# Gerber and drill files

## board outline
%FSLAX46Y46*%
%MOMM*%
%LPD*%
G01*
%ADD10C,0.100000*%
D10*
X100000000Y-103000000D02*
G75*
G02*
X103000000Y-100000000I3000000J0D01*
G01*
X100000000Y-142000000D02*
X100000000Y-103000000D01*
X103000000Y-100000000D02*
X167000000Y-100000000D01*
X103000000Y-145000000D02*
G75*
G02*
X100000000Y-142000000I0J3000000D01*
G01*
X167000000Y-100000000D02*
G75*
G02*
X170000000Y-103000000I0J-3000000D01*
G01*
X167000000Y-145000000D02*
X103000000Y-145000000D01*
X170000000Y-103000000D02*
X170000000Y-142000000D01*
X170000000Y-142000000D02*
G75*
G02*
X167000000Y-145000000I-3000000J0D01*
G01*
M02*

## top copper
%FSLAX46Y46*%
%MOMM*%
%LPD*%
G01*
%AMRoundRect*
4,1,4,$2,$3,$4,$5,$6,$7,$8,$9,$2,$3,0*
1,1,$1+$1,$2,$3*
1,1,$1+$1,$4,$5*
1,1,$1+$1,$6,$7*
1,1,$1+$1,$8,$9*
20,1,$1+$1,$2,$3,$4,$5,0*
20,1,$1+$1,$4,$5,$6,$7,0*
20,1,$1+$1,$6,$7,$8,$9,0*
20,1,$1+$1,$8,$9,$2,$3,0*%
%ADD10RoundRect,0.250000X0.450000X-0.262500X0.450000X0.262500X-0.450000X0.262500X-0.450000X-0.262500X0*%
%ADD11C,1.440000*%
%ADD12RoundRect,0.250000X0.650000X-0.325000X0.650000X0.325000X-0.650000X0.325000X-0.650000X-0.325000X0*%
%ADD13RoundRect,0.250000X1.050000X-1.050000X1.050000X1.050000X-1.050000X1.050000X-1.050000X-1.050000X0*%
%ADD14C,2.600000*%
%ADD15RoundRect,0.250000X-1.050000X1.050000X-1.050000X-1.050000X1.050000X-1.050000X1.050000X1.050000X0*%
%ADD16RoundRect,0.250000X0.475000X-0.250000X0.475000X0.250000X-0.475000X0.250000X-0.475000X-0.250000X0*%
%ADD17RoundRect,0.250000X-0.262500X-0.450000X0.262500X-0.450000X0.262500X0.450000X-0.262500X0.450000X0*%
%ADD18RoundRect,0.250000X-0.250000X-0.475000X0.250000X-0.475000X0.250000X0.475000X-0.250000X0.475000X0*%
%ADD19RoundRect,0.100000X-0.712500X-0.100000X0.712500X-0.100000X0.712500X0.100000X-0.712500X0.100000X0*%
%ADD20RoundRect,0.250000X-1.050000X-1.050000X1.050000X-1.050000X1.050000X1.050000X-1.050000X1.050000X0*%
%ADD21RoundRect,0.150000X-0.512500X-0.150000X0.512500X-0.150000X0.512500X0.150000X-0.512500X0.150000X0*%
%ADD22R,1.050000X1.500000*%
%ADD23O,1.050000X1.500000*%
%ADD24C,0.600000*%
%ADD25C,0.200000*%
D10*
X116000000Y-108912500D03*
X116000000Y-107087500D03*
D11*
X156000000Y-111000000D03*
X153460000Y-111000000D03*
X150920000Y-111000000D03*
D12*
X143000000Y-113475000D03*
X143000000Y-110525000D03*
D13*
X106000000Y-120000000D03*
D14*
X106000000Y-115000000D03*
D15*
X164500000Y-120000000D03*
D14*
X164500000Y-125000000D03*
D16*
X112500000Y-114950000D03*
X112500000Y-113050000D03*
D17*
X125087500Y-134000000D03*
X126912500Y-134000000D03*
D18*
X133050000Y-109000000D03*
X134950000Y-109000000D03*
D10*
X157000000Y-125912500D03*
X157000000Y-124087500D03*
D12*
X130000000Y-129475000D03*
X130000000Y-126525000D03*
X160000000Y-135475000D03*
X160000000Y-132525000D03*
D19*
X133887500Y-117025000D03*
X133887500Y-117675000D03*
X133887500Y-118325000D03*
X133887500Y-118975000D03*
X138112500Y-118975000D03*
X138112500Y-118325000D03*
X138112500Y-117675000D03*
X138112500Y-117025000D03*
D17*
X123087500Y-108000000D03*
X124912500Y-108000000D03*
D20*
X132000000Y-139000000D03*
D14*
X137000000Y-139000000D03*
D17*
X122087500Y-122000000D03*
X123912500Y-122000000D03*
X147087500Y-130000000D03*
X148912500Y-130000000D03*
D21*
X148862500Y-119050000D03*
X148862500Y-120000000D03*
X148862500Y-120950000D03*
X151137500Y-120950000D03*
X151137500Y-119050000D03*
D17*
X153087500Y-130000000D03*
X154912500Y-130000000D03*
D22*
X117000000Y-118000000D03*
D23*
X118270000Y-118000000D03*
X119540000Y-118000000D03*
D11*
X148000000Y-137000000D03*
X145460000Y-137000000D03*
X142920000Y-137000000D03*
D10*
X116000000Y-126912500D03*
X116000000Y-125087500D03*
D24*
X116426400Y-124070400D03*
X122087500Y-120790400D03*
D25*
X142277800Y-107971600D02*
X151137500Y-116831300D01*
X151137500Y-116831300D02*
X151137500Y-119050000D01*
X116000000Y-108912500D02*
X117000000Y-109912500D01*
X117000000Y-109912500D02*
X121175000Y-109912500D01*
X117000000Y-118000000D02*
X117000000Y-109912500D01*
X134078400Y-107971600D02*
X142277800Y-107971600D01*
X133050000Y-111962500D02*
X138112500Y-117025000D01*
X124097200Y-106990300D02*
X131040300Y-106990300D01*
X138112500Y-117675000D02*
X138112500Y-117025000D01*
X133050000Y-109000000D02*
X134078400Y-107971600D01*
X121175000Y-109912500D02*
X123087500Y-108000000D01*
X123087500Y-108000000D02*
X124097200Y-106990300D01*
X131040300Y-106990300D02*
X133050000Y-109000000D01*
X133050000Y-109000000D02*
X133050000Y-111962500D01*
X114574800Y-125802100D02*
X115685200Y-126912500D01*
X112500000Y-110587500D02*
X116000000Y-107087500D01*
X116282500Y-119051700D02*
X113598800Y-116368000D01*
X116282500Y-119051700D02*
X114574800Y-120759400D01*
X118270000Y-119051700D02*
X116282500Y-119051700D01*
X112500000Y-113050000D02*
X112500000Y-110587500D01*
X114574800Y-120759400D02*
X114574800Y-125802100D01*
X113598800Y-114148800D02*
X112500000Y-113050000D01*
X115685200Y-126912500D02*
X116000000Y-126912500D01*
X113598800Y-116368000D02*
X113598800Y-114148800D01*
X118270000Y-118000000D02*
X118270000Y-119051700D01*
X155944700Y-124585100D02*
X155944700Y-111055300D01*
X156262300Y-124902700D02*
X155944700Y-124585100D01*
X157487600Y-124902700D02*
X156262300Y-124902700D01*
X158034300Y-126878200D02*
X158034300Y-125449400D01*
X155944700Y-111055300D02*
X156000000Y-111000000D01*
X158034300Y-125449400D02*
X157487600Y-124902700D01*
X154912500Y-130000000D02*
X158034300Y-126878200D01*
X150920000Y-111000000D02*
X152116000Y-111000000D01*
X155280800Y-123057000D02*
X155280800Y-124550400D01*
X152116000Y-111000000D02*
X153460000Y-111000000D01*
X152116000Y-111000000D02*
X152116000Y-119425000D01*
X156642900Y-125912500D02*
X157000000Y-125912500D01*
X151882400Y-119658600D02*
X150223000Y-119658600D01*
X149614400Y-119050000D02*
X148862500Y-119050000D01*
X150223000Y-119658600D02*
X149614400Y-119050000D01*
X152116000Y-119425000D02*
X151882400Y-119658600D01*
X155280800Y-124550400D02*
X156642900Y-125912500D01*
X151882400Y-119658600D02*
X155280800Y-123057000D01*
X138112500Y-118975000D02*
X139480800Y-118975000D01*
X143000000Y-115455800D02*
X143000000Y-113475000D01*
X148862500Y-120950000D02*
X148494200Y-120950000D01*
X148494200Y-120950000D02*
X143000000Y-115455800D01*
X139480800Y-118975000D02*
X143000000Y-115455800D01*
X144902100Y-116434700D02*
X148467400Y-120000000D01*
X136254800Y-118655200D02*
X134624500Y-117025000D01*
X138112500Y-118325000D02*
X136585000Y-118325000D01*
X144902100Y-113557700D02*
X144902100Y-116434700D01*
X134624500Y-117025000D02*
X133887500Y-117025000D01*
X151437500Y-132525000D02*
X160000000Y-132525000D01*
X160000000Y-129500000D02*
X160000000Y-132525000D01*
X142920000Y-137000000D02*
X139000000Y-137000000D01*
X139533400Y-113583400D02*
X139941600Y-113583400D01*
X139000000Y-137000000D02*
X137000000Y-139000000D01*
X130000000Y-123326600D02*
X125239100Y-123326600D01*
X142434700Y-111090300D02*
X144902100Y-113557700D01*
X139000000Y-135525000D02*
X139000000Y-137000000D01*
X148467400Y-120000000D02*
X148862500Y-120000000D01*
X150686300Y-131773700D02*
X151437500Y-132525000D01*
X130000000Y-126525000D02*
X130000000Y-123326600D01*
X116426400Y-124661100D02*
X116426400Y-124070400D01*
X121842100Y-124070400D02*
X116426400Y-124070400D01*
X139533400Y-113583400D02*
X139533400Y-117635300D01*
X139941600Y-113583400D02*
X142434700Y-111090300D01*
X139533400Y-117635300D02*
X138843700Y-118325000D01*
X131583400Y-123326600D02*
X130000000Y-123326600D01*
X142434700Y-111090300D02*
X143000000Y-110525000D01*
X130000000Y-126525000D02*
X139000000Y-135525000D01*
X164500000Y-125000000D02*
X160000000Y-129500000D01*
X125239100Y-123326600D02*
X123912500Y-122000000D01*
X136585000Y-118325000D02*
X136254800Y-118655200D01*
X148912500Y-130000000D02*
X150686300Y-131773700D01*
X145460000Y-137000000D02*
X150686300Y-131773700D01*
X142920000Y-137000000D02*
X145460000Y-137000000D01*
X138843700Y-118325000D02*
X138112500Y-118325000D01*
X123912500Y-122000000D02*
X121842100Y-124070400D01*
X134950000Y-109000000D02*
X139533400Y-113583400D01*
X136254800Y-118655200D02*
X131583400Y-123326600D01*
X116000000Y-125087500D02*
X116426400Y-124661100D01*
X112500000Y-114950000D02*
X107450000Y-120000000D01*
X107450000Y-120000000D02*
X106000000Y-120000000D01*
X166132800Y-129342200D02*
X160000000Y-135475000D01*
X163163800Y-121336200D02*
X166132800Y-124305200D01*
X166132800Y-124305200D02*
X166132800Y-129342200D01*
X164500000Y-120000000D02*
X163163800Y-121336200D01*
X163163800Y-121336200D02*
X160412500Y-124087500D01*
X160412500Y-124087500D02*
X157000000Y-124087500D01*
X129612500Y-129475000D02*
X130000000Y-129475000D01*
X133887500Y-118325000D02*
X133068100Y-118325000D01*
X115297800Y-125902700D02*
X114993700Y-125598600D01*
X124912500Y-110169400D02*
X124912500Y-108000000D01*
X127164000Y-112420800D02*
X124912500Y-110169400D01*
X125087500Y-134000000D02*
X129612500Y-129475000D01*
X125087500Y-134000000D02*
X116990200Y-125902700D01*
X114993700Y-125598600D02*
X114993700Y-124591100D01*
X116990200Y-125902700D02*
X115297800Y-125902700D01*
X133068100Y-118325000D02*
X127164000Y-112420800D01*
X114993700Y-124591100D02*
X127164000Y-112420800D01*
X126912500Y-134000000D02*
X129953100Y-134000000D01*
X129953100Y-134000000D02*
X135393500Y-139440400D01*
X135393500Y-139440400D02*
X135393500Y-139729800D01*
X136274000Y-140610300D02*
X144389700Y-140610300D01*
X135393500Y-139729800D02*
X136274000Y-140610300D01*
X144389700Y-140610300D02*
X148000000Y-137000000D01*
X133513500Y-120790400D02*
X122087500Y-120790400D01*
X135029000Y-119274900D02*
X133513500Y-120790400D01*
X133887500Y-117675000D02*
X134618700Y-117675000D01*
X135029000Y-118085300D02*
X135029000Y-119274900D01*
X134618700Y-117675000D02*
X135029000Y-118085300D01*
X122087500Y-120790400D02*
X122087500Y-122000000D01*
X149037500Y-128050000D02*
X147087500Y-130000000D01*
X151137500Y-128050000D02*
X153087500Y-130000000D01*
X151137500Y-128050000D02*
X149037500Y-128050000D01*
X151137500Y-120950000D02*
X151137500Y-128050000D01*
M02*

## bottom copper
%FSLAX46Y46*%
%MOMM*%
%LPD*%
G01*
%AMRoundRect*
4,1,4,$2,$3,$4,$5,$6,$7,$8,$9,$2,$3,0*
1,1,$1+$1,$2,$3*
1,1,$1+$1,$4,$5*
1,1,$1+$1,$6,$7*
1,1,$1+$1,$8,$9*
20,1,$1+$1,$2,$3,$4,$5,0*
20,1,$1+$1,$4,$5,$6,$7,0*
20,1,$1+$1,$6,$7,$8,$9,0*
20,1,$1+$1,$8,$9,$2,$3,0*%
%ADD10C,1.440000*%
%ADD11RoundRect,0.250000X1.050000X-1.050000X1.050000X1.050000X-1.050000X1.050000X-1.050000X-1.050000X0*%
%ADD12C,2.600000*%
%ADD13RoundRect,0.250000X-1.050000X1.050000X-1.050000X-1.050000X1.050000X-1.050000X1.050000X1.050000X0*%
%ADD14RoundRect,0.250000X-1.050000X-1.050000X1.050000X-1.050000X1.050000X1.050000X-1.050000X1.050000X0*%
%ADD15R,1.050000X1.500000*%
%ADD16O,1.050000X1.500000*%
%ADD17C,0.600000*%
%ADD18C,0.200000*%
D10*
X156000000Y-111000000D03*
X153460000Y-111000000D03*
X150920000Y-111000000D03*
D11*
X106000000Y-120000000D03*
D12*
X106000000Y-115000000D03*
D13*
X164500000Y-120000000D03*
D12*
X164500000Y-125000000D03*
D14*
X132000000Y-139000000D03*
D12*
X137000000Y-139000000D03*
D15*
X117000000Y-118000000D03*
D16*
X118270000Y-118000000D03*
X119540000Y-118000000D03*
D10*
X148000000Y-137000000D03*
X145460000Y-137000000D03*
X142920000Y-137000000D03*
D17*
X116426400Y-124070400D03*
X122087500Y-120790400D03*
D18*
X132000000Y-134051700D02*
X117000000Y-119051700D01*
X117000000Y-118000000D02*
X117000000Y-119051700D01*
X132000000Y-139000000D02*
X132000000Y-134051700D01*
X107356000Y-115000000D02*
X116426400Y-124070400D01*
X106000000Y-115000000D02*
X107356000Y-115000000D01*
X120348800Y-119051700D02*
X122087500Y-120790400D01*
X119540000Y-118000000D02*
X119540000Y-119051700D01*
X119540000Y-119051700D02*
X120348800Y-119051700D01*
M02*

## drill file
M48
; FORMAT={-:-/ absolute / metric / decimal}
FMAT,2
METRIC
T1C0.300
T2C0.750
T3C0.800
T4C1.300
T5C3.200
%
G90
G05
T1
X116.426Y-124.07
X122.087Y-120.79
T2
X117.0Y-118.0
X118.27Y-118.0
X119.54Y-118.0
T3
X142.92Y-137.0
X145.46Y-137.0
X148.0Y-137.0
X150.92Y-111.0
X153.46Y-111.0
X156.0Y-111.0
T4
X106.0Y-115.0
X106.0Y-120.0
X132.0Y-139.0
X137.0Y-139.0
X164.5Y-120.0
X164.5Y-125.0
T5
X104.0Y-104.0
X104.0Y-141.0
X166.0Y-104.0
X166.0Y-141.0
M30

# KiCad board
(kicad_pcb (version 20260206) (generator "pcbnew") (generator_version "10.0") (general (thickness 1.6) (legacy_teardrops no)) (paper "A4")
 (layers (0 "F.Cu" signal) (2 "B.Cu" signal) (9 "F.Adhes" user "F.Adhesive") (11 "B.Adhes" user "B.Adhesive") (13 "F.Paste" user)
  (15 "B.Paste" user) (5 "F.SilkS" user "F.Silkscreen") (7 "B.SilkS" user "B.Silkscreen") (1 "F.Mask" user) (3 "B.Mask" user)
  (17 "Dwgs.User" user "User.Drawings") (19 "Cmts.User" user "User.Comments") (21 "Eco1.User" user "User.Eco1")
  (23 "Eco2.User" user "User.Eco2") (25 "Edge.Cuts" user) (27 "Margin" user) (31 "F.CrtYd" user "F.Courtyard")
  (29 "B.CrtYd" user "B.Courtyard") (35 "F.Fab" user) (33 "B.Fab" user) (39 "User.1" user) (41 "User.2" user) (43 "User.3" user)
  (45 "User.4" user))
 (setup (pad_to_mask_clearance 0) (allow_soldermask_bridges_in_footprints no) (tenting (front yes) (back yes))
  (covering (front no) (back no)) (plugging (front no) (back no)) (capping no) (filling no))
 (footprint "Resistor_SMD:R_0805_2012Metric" (layer "F.Cu") (at 116 108 90)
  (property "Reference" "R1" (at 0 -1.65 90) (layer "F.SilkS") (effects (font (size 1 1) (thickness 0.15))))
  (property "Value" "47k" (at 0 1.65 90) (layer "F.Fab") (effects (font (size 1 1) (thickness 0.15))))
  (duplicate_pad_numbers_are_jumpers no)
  (pad "1" smd roundrect (at -0.9125 0 90) (size 1.025 1.4) (layers "F.Cu" "F.Mask" "F.Paste") (roundrect_rratio 0.243902) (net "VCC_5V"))
  (pad "2" smd roundrect (at 0.9125 0 90) (size 1.025 1.4) (layers "F.Cu" "F.Mask" "F.Paste") (roundrect_rratio 0.243902) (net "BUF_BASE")))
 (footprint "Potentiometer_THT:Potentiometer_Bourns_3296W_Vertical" (layer "F.Cu") (at 156 111)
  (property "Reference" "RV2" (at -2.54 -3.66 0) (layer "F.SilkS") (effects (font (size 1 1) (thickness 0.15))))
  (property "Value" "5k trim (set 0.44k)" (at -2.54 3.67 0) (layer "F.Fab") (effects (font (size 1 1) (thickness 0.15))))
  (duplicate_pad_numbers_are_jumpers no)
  (pad "1" thru_hole circle (at 0 0) (size 1.44 1.44) (drill 0.8) (layers "*.Cu" "*.Mask") (remove_unused_layers no) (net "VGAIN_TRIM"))
  (pad "2" thru_hole circle (at -2.54 0) (size 1.44 1.44) (drill 0.8) (layers "*.Cu" "*.Mask") (remove_unused_layers no) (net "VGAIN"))
  (pad "3" thru_hole circle (at -5.08 0) (size 1.44 1.44) (drill 0.8) (layers "*.Cu" "*.Mask") (remove_unused_layers no) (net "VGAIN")))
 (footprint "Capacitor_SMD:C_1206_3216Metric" (layer "F.Cu") (at 143 112 90)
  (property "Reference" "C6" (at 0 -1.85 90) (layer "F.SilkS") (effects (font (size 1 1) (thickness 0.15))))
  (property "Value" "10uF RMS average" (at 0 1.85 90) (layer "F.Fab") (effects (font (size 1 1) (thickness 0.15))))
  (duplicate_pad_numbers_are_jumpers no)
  (pad "1" smd roundrect (at -1.475 0 90) (size 1.15 1.8) (layers "F.Cu" "F.Mask" "F.Paste") (roundrect_rratio 0.217391) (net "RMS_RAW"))
  (pad "2" smd roundrect (at 1.475 0 90) (size 1.15 1.8) (layers "F.Cu" "F.Mask" "F.Paste") (roundrect_rratio 0.217391) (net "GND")))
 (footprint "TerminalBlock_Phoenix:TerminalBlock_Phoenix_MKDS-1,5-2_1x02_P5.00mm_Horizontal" (layer "F.Cu") (at 106 120 90)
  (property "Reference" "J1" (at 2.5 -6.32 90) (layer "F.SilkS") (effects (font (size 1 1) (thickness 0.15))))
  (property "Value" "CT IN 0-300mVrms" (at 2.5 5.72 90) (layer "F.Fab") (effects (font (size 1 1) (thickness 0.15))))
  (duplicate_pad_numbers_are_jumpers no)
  (pad "1" thru_hole roundrect (at 0 0 90) (size 2.6 2.6) (drill 1.3) (layers "*.Cu" "*.Mask") (remove_unused_layers no)
   (roundrect_rratio 0.096154) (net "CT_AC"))
  (pad "2" thru_hole circle (at 5 0 90) (size 2.6 2.6) (drill 1.3) (layers "*.Cu" "*.Mask") (remove_unused_layers no) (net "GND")))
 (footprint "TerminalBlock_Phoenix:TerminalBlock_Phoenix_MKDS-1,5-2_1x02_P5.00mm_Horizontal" (layer "F.Cu") (at 164.5 120 -90)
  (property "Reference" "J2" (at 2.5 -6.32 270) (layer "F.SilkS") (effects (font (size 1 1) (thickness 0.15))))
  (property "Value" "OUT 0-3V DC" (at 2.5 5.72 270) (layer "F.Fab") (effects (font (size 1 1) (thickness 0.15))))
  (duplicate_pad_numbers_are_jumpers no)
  (pad "1" thru_hole roundrect (at 0 0 270) (size 2.6 2.6) (drill 1.3) (layers "*.Cu" "*.Mask") (remove_unused_layers no)
   (roundrect_rratio 0.096154) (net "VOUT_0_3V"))
  (pad "2" thru_hole circle (at 5 0 270) (size 2.6 2.6) (drill 1.3) (layers "*.Cu" "*.Mask") (remove_unused_layers no) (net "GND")))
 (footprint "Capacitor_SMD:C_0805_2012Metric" (layer "F.Cu") (at 112.5 114 90)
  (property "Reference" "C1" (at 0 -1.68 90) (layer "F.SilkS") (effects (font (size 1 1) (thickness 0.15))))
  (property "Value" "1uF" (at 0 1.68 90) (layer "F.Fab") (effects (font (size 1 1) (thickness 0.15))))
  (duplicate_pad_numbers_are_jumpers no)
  (pad "1" smd roundrect (at -0.95 0 90) (size 1 1.45) (layers "F.Cu" "F.Mask" "F.Paste") (roundrect_rratio 0.25) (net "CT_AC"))
  (pad "2" smd roundrect (at 0.95 0 90) (size 1 1.45) (layers "F.Cu" "F.Mask" "F.Paste") (roundrect_rratio 0.25) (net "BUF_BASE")))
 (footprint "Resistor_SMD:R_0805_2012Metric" (layer "F.Cu") (at 126 134)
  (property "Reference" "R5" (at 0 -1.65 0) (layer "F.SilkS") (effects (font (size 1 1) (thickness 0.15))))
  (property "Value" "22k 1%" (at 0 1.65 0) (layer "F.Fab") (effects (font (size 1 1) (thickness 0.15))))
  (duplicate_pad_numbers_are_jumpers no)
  (pad "1" smd roundrect (at -0.9125 0) (size 1.025 1.4) (layers "F.Cu" "F.Mask" "F.Paste") (roundrect_rratio 0.243902) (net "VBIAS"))
  (pad "2" smd roundrect (at 0.9125 0) (size 1.025 1.4) (layers "F.Cu" "F.Mask" "F.Paste") (roundrect_rratio 0.243902) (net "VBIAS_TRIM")))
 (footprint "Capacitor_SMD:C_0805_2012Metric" (layer "F.Cu") (at 134 109)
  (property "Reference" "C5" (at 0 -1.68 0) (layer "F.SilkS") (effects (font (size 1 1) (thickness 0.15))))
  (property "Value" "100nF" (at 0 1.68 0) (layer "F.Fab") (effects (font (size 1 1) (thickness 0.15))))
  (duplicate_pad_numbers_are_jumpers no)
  (pad "1" smd roundrect (at -0.95 0) (size 1 1.45) (layers "F.Cu" "F.Mask" "F.Paste") (roundrect_rratio 0.25) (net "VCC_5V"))
  (pad "2" smd roundrect (at 0.95 0) (size 1 1.45) (layers "F.Cu" "F.Mask" "F.Paste") (roundrect_rratio 0.25) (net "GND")))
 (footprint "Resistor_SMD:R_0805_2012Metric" (layer "F.Cu") (at 157 125 90)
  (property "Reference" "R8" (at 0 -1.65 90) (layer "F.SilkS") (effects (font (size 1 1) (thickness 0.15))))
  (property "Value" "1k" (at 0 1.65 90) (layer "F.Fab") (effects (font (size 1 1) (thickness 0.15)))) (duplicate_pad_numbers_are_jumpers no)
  (pad "1" smd roundrect (at -0.9125 0 90) (size 1.025 1.4) (layers "F.Cu" "F.Mask" "F.Paste") (roundrect_rratio 0.243902) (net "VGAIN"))
  (pad "2" smd roundrect (at 0.9125 0 90) (size 1.025 1.4) (layers "F.Cu" "F.Mask" "F.Paste") (roundrect_rratio 0.243902) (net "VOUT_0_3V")))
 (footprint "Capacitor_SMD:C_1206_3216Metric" (layer "F.Cu") (at 130 128 90)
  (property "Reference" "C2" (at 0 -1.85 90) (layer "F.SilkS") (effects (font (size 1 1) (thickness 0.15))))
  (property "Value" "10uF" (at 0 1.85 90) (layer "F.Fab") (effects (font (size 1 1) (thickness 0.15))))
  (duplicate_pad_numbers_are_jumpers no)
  (pad "1" smd roundrect (at -1.475 0 90) (size 1.15 1.8) (layers "F.Cu" "F.Mask" "F.Paste") (roundrect_rratio 0.217391) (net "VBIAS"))
  (pad "2" smd roundrect (at 1.475 0 90) (size 1.15 1.8) (layers "F.Cu" "F.Mask" "F.Paste") (roundrect_rratio 0.217391) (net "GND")))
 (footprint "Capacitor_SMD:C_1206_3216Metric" (layer "F.Cu") (at 160 134 90)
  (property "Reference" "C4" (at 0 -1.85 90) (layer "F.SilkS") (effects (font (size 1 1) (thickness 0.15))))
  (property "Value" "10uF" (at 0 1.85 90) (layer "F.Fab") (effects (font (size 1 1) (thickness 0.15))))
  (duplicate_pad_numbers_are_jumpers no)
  (pad "1" smd roundrect (at -1.475 0 90) (size 1.15 1.8) (layers "F.Cu" "F.Mask" "F.Paste") (roundrect_rratio 0.217391) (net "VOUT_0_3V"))
  (pad "2" smd roundrect (at 1.475 0 90) (size 1.15 1.8) (layers "F.Cu" "F.Mask" "F.Paste") (roundrect_rratio 0.217391) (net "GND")))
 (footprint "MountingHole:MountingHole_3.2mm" (layer "F.Cu") (at 166 141)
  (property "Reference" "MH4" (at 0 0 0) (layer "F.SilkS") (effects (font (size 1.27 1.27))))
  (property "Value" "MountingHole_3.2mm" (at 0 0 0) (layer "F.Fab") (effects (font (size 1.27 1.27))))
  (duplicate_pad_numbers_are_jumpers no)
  (pad "" np_thru_hole circle (at 0 0) (size 4.2 4.2) (drill 3.2) (layers "*.Mask")))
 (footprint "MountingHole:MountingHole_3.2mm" (layer "F.Cu") (at 104 104)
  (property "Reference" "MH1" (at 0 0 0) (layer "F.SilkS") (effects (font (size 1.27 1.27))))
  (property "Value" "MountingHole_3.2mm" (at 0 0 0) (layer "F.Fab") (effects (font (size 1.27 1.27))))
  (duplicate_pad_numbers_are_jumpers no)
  (pad "" np_thru_hole circle (at 0 0) (size 4.2 4.2) (drill 3.2) (layers "*.Mask")))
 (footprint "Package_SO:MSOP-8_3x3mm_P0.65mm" (layer "F.Cu") (at 136 118)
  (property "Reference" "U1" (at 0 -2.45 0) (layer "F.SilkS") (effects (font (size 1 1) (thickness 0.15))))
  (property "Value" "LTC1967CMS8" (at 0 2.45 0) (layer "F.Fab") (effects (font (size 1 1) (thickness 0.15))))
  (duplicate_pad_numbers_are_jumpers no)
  (pad "1" smd roundrect (at -2.1125 -0.975) (size 1.625 0.4) (layers "F.Cu" "F.Mask" "F.Paste") (roundrect_rratio 0.25) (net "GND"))
  (pad "2" smd roundrect (at -2.1125 -0.325) (size 1.625 0.4) (layers "F.Cu" "F.Mask" "F.Paste") (roundrect_rratio 0.25) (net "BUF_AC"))
  (pad "3" smd roundrect (at -2.1125 0.325) (size 1.625 0.4) (layers "F.Cu" "F.Mask" "F.Paste") (roundrect_rratio 0.25) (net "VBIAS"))
  (pad "4" smd roundrect (at -2.1125 0.975) (size 1.625 0.4) (layers "F.Cu" "F.Mask" "F.Paste") (roundrect_rratio 0.25))
  (pad "5" smd roundrect (at 2.1125 0.975) (size 1.625 0.4) (layers "F.Cu" "F.Mask" "F.Paste") (roundrect_rratio 0.25) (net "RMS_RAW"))
  (pad "6" smd roundrect (at 2.1125 0.325) (size 1.625 0.4) (layers "F.Cu" "F.Mask" "F.Paste") (roundrect_rratio 0.25) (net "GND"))
  (pad "7" smd roundrect (at 2.1125 -0.325) (size 1.625 0.4) (layers "F.Cu" "F.Mask" "F.Paste") (roundrect_rratio 0.25) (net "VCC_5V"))
  (pad "8" smd roundrect (at 2.1125 -0.975) (size 1.625 0.4) (layers "F.Cu" "F.Mask" "F.Paste") (roundrect_rratio 0.25) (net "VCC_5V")))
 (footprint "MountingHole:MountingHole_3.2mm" (layer "F.Cu") (at 104 141)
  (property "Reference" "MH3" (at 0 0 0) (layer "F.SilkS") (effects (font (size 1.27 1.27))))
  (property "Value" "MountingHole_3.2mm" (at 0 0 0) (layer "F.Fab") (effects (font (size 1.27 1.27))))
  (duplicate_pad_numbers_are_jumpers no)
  (pad "" np_thru_hole circle (at 0 0) (size 4.2 4.2) (drill 3.2) (layers "*.Mask")))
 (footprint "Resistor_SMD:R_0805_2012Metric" (layer "F.Cu") (at 124 108)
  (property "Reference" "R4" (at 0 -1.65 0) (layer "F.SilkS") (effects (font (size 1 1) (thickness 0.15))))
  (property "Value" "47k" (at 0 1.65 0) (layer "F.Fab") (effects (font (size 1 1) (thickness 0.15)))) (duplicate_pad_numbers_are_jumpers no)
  (pad "1" smd roundrect (at -0.9125 0) (size 1.025 1.4) (layers "F.Cu" "F.Mask" "F.Paste") (roundrect_rratio 0.243902) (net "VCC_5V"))
  (pad "2" smd roundrect (at 0.9125 0) (size 1.025 1.4) (layers "F.Cu" "F.Mask" "F.Paste") (roundrect_rratio 0.243902) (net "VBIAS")))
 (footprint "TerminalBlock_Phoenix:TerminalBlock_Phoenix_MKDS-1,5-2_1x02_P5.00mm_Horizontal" (layer "F.Cu") (at 132 139)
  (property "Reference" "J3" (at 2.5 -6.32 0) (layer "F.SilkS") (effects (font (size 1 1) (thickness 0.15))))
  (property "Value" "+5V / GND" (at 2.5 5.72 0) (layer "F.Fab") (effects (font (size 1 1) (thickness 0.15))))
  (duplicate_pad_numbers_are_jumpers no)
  (pad "1" thru_hole roundrect (at 0 0) (size 2.6 2.6) (drill 1.3) (layers "*.Cu" "*.Mask") (remove_unused_layers no)
   (roundrect_rratio 0.096154) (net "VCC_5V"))
  (pad "2" thru_hole circle (at 5 0) (size 2.6 2.6) (drill 1.3) (layers "*.Cu" "*.Mask") (remove_unused_layers no) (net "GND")))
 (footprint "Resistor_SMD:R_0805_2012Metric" (layer "F.Cu") (at 123 122)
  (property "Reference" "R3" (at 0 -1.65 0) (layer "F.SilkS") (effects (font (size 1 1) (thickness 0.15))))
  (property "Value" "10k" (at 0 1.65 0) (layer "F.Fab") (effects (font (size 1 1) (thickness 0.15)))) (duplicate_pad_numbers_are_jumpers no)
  (pad "1" smd roundrect (at -0.9125 0) (size 1.025 1.4) (layers "F.Cu" "F.Mask" "F.Paste") (roundrect_rratio 0.243902) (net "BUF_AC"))
  (pad "2" smd roundrect (at 0.9125 0) (size 1.025 1.4) (layers "F.Cu" "F.Mask" "F.Paste") (roundrect_rratio 0.243902) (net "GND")))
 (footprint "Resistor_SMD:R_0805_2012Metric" (layer "F.Cu") (at 148 130)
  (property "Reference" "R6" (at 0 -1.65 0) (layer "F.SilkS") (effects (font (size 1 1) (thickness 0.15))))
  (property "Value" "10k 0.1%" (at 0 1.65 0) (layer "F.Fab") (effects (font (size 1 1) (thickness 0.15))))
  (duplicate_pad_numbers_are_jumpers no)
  (pad "1" smd roundrect (at -0.9125 0) (size 1.025 1.4) (layers "F.Cu" "F.Mask" "F.Paste") (roundrect_rratio 0.243902) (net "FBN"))
  (pad "2" smd roundrect (at 0.9125 0) (size 1.025 1.4) (layers "F.Cu" "F.Mask" "F.Paste") (roundrect_rratio 0.243902) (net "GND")))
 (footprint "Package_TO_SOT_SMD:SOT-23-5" (layer "F.Cu") (at 150 120)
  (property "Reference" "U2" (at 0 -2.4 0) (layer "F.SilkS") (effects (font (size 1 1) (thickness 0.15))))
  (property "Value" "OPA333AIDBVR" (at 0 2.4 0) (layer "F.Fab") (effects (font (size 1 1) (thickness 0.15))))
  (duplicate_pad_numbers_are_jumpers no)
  (pad "1" smd roundrect (at -1.1375 -0.95) (size 1.325 0.6) (layers "F.Cu" "F.Mask" "F.Paste") (roundrect_rratio 0.25) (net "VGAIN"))
  (pad "2" smd roundrect (at -1.1375 0) (size 1.325 0.6) (layers "F.Cu" "F.Mask" "F.Paste") (roundrect_rratio 0.25) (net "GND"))
  (pad "3" smd roundrect (at -1.1375 0.95) (size 1.325 0.6) (layers "F.Cu" "F.Mask" "F.Paste") (roundrect_rratio 0.25) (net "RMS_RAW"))
  (pad "4" smd roundrect (at 1.1375 0.95) (size 1.325 0.6) (layers "F.Cu" "F.Mask" "F.Paste") (roundrect_rratio 0.25) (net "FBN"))
  (pad "5" smd roundrect (at 1.1375 -0.95) (size 1.325 0.6) (layers "F.Cu" "F.Mask" "F.Paste") (roundrect_rratio 0.25) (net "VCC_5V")))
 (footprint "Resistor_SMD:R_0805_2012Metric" (layer "F.Cu") (at 154 130)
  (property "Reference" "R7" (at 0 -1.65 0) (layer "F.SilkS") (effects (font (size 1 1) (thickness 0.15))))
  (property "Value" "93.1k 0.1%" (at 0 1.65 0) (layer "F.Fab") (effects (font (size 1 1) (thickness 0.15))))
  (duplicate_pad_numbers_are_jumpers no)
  (pad "1" smd roundrect (at -0.9125 0) (size 1.025 1.4) (layers "F.Cu" "F.Mask" "F.Paste") (roundrect_rratio 0.243902) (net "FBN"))
  (pad "2" smd roundrect (at 0.9125 0) (size 1.025 1.4) (layers "F.Cu" "F.Mask" "F.Paste") (roundrect_rratio 0.243902) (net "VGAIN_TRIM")))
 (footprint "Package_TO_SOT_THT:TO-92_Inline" (layer "F.Cu") (at 117 118)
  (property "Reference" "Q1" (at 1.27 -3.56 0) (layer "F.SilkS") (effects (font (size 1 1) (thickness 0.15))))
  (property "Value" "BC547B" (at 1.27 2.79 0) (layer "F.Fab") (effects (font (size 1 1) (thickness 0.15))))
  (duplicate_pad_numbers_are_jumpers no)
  (pad "1" thru_hole rect (at 0 0) (size 1.05 1.5) (drill 0.75) (layers "*.Cu" "*.Mask") (remove_unused_layers no) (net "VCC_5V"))
  (pad "2" thru_hole oval (at 1.27 0) (size 1.05 1.5) (drill 0.75) (layers "*.Cu" "*.Mask") (remove_unused_layers no) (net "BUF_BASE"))
  (pad "3" thru_hole oval (at 2.54 0) (size 1.05 1.5) (drill 0.75) (layers "*.Cu" "*.Mask") (remove_unused_layers no) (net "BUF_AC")))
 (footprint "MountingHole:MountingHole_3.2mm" (layer "F.Cu") (at 166 104)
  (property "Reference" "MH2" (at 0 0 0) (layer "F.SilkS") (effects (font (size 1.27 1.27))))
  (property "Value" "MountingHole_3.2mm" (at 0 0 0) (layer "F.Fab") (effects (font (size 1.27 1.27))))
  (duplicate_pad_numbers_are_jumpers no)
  (pad "" np_thru_hole circle (at 0 0) (size 4.2 4.2) (drill 3.2) (layers "*.Mask")))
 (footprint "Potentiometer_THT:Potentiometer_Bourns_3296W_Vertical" (layer "F.Cu") (at 148 137)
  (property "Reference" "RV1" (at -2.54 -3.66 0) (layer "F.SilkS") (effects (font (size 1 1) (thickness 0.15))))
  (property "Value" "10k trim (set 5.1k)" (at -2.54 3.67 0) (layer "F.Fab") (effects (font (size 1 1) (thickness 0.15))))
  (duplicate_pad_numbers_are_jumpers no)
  (pad "1" thru_hole circle (at 0 0) (size 1.44 1.44) (drill 0.8) (layers "*.Cu" "*.Mask") (remove_unused_layers no) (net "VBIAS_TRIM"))
  (pad "2" thru_hole circle (at -2.54 0) (size 1.44 1.44) (drill 0.8) (layers "*.Cu" "*.Mask") (remove_unused_layers no) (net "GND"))
  (pad "3" thru_hole circle (at -5.08 0) (size 1.44 1.44) (drill 0.8) (layers "*.Cu" "*.Mask") (remove_unused_layers no) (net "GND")))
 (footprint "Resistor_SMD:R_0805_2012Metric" (layer "F.Cu") (at 116 126 90)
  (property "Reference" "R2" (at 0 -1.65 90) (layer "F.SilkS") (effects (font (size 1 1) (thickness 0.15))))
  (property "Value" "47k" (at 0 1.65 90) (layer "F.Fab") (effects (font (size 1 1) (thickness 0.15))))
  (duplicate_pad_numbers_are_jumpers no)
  (pad "1" smd roundrect (at -0.9125 0 90) (size 1.025 1.4) (layers "F.Cu" "F.Mask" "F.Paste") (roundrect_rratio 0.243902) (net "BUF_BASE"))
  (pad "2" smd roundrect (at 0.9125 0 90) (size 1.025 1.4) (layers "F.Cu" "F.Mask" "F.Paste") (roundrect_rratio 0.243902) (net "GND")))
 (gr_arc (start 100 103) (mid 100.87868 100.87868) (end 103 100) (stroke (width 0.1) (type default)) (layer "Edge.Cuts"))
 (gr_line (start 100 142) (end 100 103) (stroke (width 0.1) (type default)) (layer "Edge.Cuts"))
 (gr_line (start 103 100) (end 167 100) (stroke (width 0.1) (type default)) (layer "Edge.Cuts"))
 (gr_arc (start 103 145) (mid 100.87868 144.12132) (end 100 142) (stroke (width 0.1) (type default)) (layer "Edge.Cuts"))
 (gr_arc (start 167 100) (mid 169.12132 100.87868) (end 170 103) (stroke (width 0.1) (type default)) (layer "Edge.Cuts"))
 (gr_line (start 167 145) (end 103 145) (stroke (width 0.1) (type default)) (layer "Edge.Cuts"))
 (gr_line (start 170 103) (end 170 142) (stroke (width 0.1) (type default)) (layer "Edge.Cuts"))
 (gr_arc (start 170 142) (mid 169.12132 144.12132) (end 167 145) (stroke (width 0.1) (type default)) (layer "Edge.Cuts"))
 (segment (start 142.2778 107.9716) (end 151.1375 116.8313) (width 0.2) (layer "F.Cu") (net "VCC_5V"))
 (segment (start 151.1375 116.8313) (end 151.1375 119.05) (width 0.2) (layer "F.Cu") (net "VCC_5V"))
 (segment (start 116 108.9125) (end 117 109.9125) (width 0.2) (layer "F.Cu") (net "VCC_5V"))
 (segment (start 117 109.9125) (end 121.175 109.9125) (width 0.2) (layer "F.Cu") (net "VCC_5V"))
 (segment (start 117 118) (end 117 109.9125) (width 0.2) (layer "F.Cu") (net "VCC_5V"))
 (segment (start 134.0784 107.9716) (end 142.2778 107.9716) (width 0.2) (layer "F.Cu") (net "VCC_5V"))
 (segment (start 133.05 111.9625) (end 138.1125 117.025) (width 0.2) (layer "F.Cu") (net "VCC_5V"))
 (segment (start 124.0972 106.9903) (end 131.0403 106.9903) (width 0.2) (layer "F.Cu") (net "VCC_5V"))
 (segment (start 138.1125 117.675) (end 138.1125 117.025) (width 0.2) (layer "F.Cu") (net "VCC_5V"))
 (segment (start 133.05 109) (end 134.0784 107.9716) (width 0.2) (layer "F.Cu") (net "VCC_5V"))
 (segment (start 121.175 109.9125) (end 123.0875 108) (width 0.2) (layer "F.Cu") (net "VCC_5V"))
 (segment (start 123.0875 108) (end 124.0972 106.9903) (width 0.2) (layer "F.Cu") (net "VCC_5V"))
 (segment (start 131.0403 106.9903) (end 133.05 109) (width 0.2) (layer "F.Cu") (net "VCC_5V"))
 (segment (start 133.05 109) (end 133.05 111.9625) (width 0.2) (layer "F.Cu") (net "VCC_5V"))
 (segment (start 132 134.0517) (end 117 119.0517) (width 0.2) (layer "B.Cu") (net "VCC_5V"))
 (segment (start 117 118) (end 117 119.0517) (width 0.2) (layer "B.Cu") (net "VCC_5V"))
 (segment (start 132 139) (end 132 134.0517) (width 0.2) (layer "B.Cu") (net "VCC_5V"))
 (segment (start 114.5748 125.8021) (end 115.6852 126.9125) (width 0.2) (layer "F.Cu") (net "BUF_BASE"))
 (segment (start 112.5 110.5875) (end 116 107.0875) (width 0.2) (layer "F.Cu") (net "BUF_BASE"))
 (segment (start 116.2825 119.0517) (end 113.5988 116.368) (width 0.2) (layer "F.Cu") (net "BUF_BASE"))
 (segment (start 116.2825 119.0517) (end 114.5748 120.7594) (width 0.2) (layer "F.Cu") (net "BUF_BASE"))
 (segment (start 118.27 119.0517) (end 116.2825 119.0517) (width 0.2) (layer "F.Cu") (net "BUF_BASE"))
 (segment (start 112.5 113.05) (end 112.5 110.5875) (width 0.2) (layer "F.Cu") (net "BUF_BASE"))
 (segment (start 114.5748 120.7594) (end 114.5748 125.8021) (width 0.2) (layer "F.Cu") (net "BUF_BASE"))
 (segment (start 113.5988 114.1488) (end 112.5 113.05) (width 0.2) (layer "F.Cu") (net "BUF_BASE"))
 (segment (start 115.6852 126.9125) (end 116 126.9125) (width 0.2) (layer "F.Cu") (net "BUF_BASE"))
 (segment (start 113.5988 116.368) (end 113.5988 114.1488) (width 0.2) (layer "F.Cu") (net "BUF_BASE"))
 (segment (start 118.27 118) (end 118.27 119.0517) (width 0.2) (layer "F.Cu") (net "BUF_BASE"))
 (segment (start 155.9447 124.5851) (end 155.9447 111.0553) (width 0.2) (layer "F.Cu") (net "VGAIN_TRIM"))
 (segment (start 156.2623 124.9027) (end 155.9447 124.5851) (width 0.2) (layer "F.Cu") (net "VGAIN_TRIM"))
 (segment (start 157.4876 124.9027) (end 156.2623 124.9027) (width 0.2) (layer "F.Cu") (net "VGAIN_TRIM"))
 (segment (start 158.0343 126.8782) (end 158.0343 125.4494) (width 0.2) (layer "F.Cu") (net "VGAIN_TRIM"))
 (segment (start 155.9447 111.0553) (end 156 111) (width 0.2) (layer "F.Cu") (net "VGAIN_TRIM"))
 (segment (start 158.0343 125.4494) (end 157.4876 124.9027) (width 0.2) (layer "F.Cu") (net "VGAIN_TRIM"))
 (segment (start 154.9125 130) (end 158.0343 126.8782) (width 0.2) (layer "F.Cu") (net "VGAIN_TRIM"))
 (segment (start 150.92 111) (end 152.116 111) (width 0.2) (layer "F.Cu") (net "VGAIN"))
 (segment (start 155.2808 123.057) (end 155.2808 124.5504) (width 0.2) (layer "F.Cu") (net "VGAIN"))
 (segment (start 152.116 111) (end 153.46 111) (width 0.2) (layer "F.Cu") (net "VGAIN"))
 (segment (start 152.116 111) (end 152.116 119.425) (width 0.2) (layer "F.Cu") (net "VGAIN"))
 (segment (start 156.6429 125.9125) (end 157 125.9125) (width 0.2) (layer "F.Cu") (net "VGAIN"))
 (segment (start 151.8824 119.6586) (end 150.223 119.6586) (width 0.2) (layer "F.Cu") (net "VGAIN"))
 (segment (start 149.6144 119.05) (end 148.8625 119.05) (width 0.2) (layer "F.Cu") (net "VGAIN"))
 (segment (start 150.223 119.6586) (end 149.6144 119.05) (width 0.2) (layer "F.Cu") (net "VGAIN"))
 (segment (start 152.116 119.425) (end 151.8824 119.6586) (width 0.2) (layer "F.Cu") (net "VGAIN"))
 (segment (start 155.2808 124.5504) (end 156.6429 125.9125) (width 0.2) (layer "F.Cu") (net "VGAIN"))
 (segment (start 151.8824 119.6586) (end 155.2808 123.057) (width 0.2) (layer "F.Cu") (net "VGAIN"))
 (segment (start 138.1125 118.975) (end 139.4808 118.975) (width 0.2) (layer "F.Cu") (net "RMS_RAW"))
 (segment (start 143 115.4558) (end 143 113.475) (width 0.2) (layer "F.Cu") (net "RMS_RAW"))
 (segment (start 148.8625 120.95) (end 148.4942 120.95) (width 0.2) (layer "F.Cu") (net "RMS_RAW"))
 (segment (start 148.4942 120.95) (end 143 115.4558) (width 0.2) (layer "F.Cu") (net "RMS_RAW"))
 (segment (start 139.4808 118.975) (end 143 115.4558) (width 0.2) (layer "F.Cu") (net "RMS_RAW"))
 (segment (start 144.9021 116.4347) (end 148.4674 120) (width 0.2) (layer "F.Cu") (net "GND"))
 (segment (start 136.2548 118.6552) (end 134.6245 117.025) (width 0.2) (layer "F.Cu") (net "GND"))
 (segment (start 138.1125 118.325) (end 136.585 118.325) (width 0.2) (layer "F.Cu") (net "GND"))
 (segment (start 144.9021 113.5577) (end 144.9021 116.4347) (width 0.2) (layer "F.Cu") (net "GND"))
 (segment (start 134.6245 117.025) (end 133.8875 117.025) (width 0.2) (layer "F.Cu") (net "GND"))
 (segment (start 151.4375 132.525) (end 160 132.525) (width 0.2) (layer "F.Cu") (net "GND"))
 (segment (start 160 129.5) (end 160 132.525) (width 0.2) (layer "F.Cu") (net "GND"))
 (segment (start 142.92 137) (end 139 137) (width 0.2) (layer "F.Cu") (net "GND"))
 (segment (start 139.5334 113.5834) (end 139.9416 113.5834) (width 0.2) (layer "F.Cu") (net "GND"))
 (segment (start 139 137) (end 137 139) (width 0.2) (layer "F.Cu") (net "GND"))
 (segment (start 130 123.3266) (end 125.2391 123.3266) (width 0.2) (layer "F.Cu") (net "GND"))
 (segment (start 142.4347 111.0903) (end 144.9021 113.5577) (width 0.2) (layer "F.Cu") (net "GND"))
 (segment (start 139 135.525) (end 139 137) (width 0.2) (layer "F.Cu") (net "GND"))
 (segment (start 148.4674 120) (end 148.8625 120) (width 0.2) (layer "F.Cu") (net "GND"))
 (segment (start 150.6863 131.7737) (end 151.4375 132.525) (width 0.2) (layer "F.Cu") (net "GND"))
 (segment (start 130 126.525) (end 130 123.3266) (width 0.2) (layer "F.Cu") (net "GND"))
 (segment (start 116.4264 124.6611) (end 116.4264 124.0704) (width 0.2) (layer "F.Cu") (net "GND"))
 (segment (start 121.8421 124.0704) (end 116.4264 124.0704) (width 0.2) (layer "F.Cu") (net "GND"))
 (segment (start 139.5334 113.5834) (end 139.5334 117.6353) (width 0.2) (layer "F.Cu") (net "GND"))
 (segment (start 139.9416 113.5834) (end 142.4347 111.0903) (width 0.2) (layer "F.Cu") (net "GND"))
 (segment (start 139.5334 117.6353) (end 138.8437 118.325) (width 0.2) (layer "F.Cu") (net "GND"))
 (segment (start 131.5834 123.3266) (end 130 123.3266) (width 0.2) (layer "F.Cu") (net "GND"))
 (segment (start 142.4347 111.0903) (end 143 110.525) (width 0.2) (layer "F.Cu") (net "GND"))
 (segment (start 130 126.525) (end 139 135.525) (width 0.2) (layer "F.Cu") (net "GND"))
 (segment (start 164.5 125) (end 160 129.5) (width 0.2) (layer "F.Cu") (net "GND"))
 (segment (start 125.2391 123.3266) (end 123.9125 122) (width 0.2) (layer "F.Cu") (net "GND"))
 (segment (start 136.585 118.325) (end 136.2548 118.6552) (width 0.2) (layer "F.Cu") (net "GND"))
 (segment (start 148.9125 130) (end 150.6863 131.7737) (width 0.2) (layer "F.Cu") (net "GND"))
 (segment (start 145.46 137) (end 150.6863 131.7737) (width 0.2) (layer "F.Cu") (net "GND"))
 (segment (start 142.92 137) (end 145.46 137) (width 0.2) (layer "F.Cu") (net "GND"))
 (segment (start 138.8437 118.325) (end 138.1125 118.325) (width 0.2) (layer "F.Cu") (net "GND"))
 (segment (start 123.9125 122) (end 121.8421 124.0704) (width 0.2) (layer "F.Cu") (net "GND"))
 (segment (start 134.95 109) (end 139.5334 113.5834) (width 0.2) (layer "F.Cu") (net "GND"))
 (segment (start 136.2548 118.6552) (end 131.5834 123.3266) (width 0.2) (layer "F.Cu") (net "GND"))
 (segment (start 116 125.0875) (end 116.4264 124.6611) (width 0.2) (layer "F.Cu") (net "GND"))
 (via (at 116.4264 124.0704) (size 0.6) (drill 0.3) (layers "F.Cu" "B.Cu") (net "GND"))
 (segment (start 107.356 115) (end 116.4264 124.0704) (width 0.2) (layer "B.Cu") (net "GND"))
 (segment (start 106 115) (end 107.356 115) (width 0.2) (layer "B.Cu") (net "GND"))
 (segment (start 112.5 114.95) (end 107.45 120) (width 0.2) (layer "F.Cu") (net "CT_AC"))
 (segment (start 107.45 120) (end 106 120) (width 0.2) (layer "F.Cu") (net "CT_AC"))
 (segment (start 166.1328 129.3422) (end 160 135.475) (width 0.2) (layer "F.Cu") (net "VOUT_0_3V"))
 (segment (start 163.1638 121.3362) (end 166.1328 124.3052) (width 0.2) (layer "F.Cu") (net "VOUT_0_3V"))
 (segment (start 166.1328 124.3052) (end 166.1328 129.3422) (width 0.2) (layer "F.Cu") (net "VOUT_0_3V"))
 (segment (start 164.5 120) (end 163.1638 121.3362) (width 0.2) (layer "F.Cu") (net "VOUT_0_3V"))
 (segment (start 163.1638 121.3362) (end 160.4125 124.0875) (width 0.2) (layer "F.Cu") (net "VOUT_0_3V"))
 (segment (start 160.4125 124.0875) (end 157 124.0875) (width 0.2) (layer "F.Cu") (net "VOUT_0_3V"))
 (segment (start 129.6125 129.475) (end 130 129.475) (width 0.2) (layer "F.Cu") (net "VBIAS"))
 (segment (start 133.8875 118.325) (end 133.0681 118.325) (width 0.2) (layer "F.Cu") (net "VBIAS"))
 (segment (start 115.2978 125.9027) (end 114.9937 125.5986) (width 0.2) (layer "F.Cu") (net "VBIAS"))
 (segment (start 124.9125 110.1694) (end 124.9125 108) (width 0.2) (layer "F.Cu") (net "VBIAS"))
 (segment (start 127.164 112.4208) (end 124.9125 110.1694) (width 0.2) (layer "F.Cu") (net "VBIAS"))
 (segment (start 125.0875 134) (end 129.6125 129.475) (width 0.2) (layer "F.Cu") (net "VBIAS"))
 (segment (start 125.0875 134) (end 116.9902 125.9027) (width 0.2) (layer "F.Cu") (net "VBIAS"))
 (segment (start 114.9937 125.5986) (end 114.9937 124.5911) (width 0.2) (layer "F.Cu") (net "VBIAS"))
 (segment (start 116.9902 125.9027) (end 115.2978 125.9027) (width 0.2) (layer "F.Cu") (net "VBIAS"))
 (segment (start 133.0681 118.325) (end 127.164 112.4208) (width 0.2) (layer "F.Cu") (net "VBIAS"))
 (segment (start 114.9937 124.5911) (end 127.164 112.4208) (width 0.2) (layer "F.Cu") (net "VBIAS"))
 (segment (start 126.9125 134) (end 129.9531 134) (width 0.2) (layer "F.Cu") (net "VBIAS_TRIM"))
 (segment (start 129.9531 134) (end 135.3935 139.4404) (width 0.2) (layer "F.Cu") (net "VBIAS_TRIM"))
 (segment (start 135.3935 139.4404) (end 135.3935 139.7298) (width 0.2) (layer "F.Cu") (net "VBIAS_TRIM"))
 (segment (start 136.274 140.6103) (end 144.3897 140.6103) (width 0.2) (layer "F.Cu") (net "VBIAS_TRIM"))
 (segment (start 135.3935 139.7298) (end 136.274 140.6103) (width 0.2) (layer "F.Cu") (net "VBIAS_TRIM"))
 (segment (start 144.3897 140.6103) (end 148 137) (width 0.2) (layer "F.Cu") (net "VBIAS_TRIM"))
 (segment (start 133.5135 120.7904) (end 122.0875 120.7904) (width 0.2) (layer "F.Cu") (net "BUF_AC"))
 (segment (start 135.029 119.2749) (end 133.5135 120.7904) (width 0.2) (layer "F.Cu") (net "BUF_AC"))
 (segment (start 133.8875 117.675) (end 134.6187 117.675) (width 0.2) (layer "F.Cu") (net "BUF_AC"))
 (segment (start 135.029 118.0853) (end 135.029 119.2749) (width 0.2) (layer "F.Cu") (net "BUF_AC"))
 (segment (start 134.6187 117.675) (end 135.029 118.0853) (width 0.2) (layer "F.Cu") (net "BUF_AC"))
 (segment (start 122.0875 120.7904) (end 122.0875 122) (width 0.2) (layer "F.Cu") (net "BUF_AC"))
 (via (at 122.0875 120.7904) (size 0.6) (drill 0.3) (layers "F.Cu" "B.Cu") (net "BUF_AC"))
 (segment (start 120.3488 119.0517) (end 122.0875 120.7904) (width 0.2) (layer "B.Cu") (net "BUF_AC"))
 (segment (start 119.54 118) (end 119.54 119.0517) (width 0.2) (layer "B.Cu") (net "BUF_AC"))
 (segment (start 119.54 119.0517) (end 120.3488 119.0517) (width 0.2) (layer "B.Cu") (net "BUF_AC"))
 (segment (start 149.0375 128.05) (end 147.0875 130) (width 0.2) (layer "F.Cu") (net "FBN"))
 (segment (start 151.1375 128.05) (end 153.0875 130) (width 0.2) (layer "F.Cu") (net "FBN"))
 (segment (start 151.1375 128.05) (end 149.0375 128.05) (width 0.2) (layer "F.Cu") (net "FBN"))
 (segment (start 151.1375 120.95) (end 151.1375 128.05) (width 0.2) (layer "F.Cu") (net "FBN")))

